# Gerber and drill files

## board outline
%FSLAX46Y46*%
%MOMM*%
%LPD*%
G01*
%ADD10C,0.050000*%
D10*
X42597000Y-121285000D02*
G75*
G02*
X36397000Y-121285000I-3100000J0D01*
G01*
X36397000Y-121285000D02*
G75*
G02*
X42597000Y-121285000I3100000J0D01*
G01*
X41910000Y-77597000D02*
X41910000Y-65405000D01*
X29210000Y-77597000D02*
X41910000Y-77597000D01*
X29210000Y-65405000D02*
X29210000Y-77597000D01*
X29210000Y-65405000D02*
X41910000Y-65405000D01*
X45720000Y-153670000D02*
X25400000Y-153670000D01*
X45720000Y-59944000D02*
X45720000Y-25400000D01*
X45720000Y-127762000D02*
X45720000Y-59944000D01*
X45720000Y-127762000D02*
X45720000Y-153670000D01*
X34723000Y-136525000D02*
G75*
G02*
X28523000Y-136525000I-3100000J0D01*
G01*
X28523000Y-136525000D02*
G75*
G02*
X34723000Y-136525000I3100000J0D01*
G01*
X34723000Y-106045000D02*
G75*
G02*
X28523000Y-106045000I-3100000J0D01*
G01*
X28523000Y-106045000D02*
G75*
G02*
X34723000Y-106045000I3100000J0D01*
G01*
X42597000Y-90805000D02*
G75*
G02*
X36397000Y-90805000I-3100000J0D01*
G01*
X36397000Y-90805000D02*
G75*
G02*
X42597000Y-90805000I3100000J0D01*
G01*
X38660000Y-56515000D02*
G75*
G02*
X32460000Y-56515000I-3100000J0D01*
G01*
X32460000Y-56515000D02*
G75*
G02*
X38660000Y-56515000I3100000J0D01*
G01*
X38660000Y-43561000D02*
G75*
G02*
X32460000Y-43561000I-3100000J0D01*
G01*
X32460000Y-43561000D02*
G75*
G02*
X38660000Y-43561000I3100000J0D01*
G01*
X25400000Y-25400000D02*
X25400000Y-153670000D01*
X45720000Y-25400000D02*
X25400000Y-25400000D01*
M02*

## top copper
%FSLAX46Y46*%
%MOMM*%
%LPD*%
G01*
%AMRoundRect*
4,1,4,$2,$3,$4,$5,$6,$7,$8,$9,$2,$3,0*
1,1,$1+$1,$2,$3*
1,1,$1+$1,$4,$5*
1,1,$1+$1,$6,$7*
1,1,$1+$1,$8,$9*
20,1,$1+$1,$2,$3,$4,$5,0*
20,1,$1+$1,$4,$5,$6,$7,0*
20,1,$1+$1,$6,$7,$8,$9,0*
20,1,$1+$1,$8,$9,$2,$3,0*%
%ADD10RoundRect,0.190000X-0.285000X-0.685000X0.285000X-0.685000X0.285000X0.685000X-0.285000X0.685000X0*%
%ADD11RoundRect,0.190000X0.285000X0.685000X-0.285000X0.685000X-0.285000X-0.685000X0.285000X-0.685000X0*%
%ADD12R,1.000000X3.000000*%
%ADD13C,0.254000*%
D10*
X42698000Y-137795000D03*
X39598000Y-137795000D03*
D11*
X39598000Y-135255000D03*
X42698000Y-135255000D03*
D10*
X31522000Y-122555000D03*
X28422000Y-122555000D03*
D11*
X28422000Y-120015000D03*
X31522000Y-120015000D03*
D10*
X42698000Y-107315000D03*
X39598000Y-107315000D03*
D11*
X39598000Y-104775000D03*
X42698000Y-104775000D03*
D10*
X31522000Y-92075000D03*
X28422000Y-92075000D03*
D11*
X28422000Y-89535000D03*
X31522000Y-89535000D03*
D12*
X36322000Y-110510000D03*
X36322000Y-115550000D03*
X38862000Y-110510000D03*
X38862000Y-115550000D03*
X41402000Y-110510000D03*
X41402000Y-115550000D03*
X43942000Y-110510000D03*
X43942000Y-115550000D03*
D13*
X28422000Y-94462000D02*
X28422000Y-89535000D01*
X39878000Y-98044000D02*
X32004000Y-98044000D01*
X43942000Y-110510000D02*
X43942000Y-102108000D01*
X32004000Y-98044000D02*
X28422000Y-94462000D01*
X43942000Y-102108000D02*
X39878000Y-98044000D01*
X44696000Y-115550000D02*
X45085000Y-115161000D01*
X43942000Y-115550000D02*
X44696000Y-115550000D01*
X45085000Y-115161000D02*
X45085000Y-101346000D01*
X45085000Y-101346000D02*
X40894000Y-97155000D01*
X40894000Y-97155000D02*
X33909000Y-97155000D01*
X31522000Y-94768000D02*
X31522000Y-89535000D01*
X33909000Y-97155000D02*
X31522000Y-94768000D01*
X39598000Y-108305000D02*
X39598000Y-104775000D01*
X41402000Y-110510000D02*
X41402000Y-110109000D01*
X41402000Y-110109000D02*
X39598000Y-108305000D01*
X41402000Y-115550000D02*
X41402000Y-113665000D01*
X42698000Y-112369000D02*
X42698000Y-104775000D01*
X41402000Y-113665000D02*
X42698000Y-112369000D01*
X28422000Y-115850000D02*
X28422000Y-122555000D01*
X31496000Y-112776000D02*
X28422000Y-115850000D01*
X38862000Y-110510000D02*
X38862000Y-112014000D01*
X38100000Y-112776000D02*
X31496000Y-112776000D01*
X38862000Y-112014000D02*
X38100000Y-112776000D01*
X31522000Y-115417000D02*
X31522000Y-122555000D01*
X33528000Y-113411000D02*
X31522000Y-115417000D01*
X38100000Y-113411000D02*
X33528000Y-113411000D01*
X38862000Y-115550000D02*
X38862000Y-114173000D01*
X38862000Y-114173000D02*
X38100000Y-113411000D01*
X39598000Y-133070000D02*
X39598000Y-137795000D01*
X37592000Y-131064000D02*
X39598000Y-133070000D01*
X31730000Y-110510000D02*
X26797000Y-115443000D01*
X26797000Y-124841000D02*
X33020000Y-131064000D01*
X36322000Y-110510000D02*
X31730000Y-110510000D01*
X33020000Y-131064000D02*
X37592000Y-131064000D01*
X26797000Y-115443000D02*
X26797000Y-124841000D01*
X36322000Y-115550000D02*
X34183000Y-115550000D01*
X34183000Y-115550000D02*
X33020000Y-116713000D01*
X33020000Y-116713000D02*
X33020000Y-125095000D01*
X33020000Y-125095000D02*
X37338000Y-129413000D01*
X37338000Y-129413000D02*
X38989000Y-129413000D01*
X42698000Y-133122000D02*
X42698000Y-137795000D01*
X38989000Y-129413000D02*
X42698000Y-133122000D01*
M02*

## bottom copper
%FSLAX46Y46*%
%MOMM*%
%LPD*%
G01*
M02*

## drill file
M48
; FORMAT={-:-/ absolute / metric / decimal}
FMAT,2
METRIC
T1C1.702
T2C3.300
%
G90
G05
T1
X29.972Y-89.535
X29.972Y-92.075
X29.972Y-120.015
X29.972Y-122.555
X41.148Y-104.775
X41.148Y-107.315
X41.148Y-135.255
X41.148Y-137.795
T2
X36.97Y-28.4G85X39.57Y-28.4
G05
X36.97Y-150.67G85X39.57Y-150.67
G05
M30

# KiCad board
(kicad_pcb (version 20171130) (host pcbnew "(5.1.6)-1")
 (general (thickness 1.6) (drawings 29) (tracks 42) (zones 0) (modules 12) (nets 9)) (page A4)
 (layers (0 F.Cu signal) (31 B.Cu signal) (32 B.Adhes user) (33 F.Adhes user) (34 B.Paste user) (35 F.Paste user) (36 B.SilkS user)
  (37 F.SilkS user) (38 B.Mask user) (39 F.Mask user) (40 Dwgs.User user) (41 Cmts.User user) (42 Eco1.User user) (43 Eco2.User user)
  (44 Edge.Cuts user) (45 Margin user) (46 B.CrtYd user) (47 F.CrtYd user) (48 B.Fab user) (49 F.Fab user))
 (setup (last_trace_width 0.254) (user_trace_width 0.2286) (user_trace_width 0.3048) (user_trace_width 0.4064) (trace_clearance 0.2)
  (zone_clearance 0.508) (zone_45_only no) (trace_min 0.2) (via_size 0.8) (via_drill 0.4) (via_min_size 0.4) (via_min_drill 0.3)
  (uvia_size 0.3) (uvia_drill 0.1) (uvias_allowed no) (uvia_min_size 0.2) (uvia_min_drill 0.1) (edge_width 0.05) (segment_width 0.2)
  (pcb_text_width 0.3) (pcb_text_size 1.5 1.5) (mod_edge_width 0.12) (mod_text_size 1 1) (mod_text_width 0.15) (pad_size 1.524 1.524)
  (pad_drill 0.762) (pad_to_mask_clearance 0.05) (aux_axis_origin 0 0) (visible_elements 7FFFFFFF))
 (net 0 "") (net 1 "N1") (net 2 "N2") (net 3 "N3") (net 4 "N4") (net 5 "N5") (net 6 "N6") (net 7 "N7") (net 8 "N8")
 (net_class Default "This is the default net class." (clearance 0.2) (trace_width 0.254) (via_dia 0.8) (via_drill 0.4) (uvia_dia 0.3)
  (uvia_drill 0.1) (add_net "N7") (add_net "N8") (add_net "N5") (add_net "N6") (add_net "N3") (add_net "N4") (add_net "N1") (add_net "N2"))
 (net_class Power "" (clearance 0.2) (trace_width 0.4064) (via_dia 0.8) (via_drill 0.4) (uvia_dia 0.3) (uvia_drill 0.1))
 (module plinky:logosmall (layer F.Cu) (at 35.687 34.417)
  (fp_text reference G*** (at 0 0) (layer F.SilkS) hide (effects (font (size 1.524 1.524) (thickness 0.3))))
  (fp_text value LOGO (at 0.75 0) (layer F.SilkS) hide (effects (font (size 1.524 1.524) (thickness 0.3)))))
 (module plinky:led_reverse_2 (layer F.Cu) (at 41.148 137.795)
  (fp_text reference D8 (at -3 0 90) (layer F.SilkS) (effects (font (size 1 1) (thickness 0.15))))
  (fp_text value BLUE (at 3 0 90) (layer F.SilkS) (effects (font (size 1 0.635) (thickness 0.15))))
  (pad "" np_thru_hole oval (at 0 0) (size 1.7018 1.7018) (drill oval 1.7018) (layers *.Cu *.Mask))
  (pad 2 smd roundrect (at 1.55 0) (size 0.95 1.75) (layers F.Cu F.Paste F.Mask) (roundrect_rratio 0.2) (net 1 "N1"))
  (pad 1 smd roundrect (at -1.55 0) (size 0.95 1.75) (layers F.Cu F.Paste F.Mask) (roundrect_rratio 0.2) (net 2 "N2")))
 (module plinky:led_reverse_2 (layer F.Cu) (at 41.148 135.255 180)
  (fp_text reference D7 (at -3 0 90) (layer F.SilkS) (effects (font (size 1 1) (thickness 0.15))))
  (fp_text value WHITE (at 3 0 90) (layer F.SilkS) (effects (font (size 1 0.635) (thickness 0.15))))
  (pad "" np_thru_hole oval (at 0 0 180) (size 1.7018 1.7018) (drill oval 1.7018) (layers *.Cu *.Mask))
  (pad 2 smd roundrect (at 1.55 0 180) (size 0.95 1.75) (layers F.Cu F.Paste F.Mask) (roundrect_rratio 0.2) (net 2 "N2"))
  (pad 1 smd roundrect (at -1.55 0 180) (size 0.95 1.75) (layers F.Cu F.Paste F.Mask) (roundrect_rratio 0.2) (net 1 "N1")))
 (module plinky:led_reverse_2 (layer F.Cu) (at 29.972 122.555)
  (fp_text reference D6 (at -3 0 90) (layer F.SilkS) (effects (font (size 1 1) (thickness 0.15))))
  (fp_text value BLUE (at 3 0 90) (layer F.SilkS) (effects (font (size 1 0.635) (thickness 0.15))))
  (pad "" np_thru_hole oval (at 0 0) (size 1.7018 1.7018) (drill oval 1.7018) (layers *.Cu *.Mask))
  (pad 2 smd roundrect (at 1.55 0) (size 0.95 1.75) (layers F.Cu F.Paste F.Mask) (roundrect_rratio 0.2) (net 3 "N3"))
  (pad 1 smd roundrect (at -1.55 0) (size 0.95 1.75) (layers F.Cu F.Paste F.Mask) (roundrect_rratio 0.2) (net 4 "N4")))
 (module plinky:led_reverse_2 (layer F.Cu) (at 29.972 120.015 180)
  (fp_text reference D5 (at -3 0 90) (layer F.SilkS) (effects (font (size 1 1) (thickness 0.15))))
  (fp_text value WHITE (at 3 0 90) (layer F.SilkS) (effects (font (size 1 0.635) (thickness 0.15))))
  (pad "" np_thru_hole oval (at 0 0 180) (size 1.7018 1.7018) (drill oval 1.7018) (layers *.Cu *.Mask))
  (pad 2 smd roundrect (at 1.55 0 180) (size 0.95 1.75) (layers F.Cu F.Paste F.Mask) (roundrect_rratio 0.2) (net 4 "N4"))
  (pad 1 smd roundrect (at -1.55 0 180) (size 0.95 1.75) (layers F.Cu F.Paste F.Mask) (roundrect_rratio 0.2) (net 3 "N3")))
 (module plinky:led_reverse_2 (layer F.Cu) (at 41.148 107.315)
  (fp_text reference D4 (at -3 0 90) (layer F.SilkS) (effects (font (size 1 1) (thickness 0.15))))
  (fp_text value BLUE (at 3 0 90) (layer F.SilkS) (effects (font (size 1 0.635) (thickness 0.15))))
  (pad "" np_thru_hole oval (at 0 0) (size 1.7018 1.7018) (drill oval 1.7018) (layers *.Cu *.Mask))
  (pad 2 smd roundrect (at 1.55 0) (size 0.95 1.75) (layers F.Cu F.Paste F.Mask) (roundrect_rratio 0.2) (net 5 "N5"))
  (pad 1 smd roundrect (at -1.55 0) (size 0.95 1.75) (layers F.Cu F.Paste F.Mask) (roundrect_rratio 0.2) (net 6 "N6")))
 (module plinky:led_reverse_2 (layer F.Cu) (at 41.148 104.775 180)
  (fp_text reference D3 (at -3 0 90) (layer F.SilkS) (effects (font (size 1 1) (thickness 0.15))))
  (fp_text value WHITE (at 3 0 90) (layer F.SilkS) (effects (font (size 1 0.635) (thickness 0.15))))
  (pad "" np_thru_hole oval (at 0 0 180) (size 1.7018 1.7018) (drill oval 1.7018) (layers *.Cu *.Mask))
  (pad 2 smd roundrect (at 1.55 0 180) (size 0.95 1.75) (layers F.Cu F.Paste F.Mask) (roundrect_rratio 0.2) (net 6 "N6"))
  (pad 1 smd roundrect (at -1.55 0 180) (size 0.95 1.75) (layers F.Cu F.Paste F.Mask) (roundrect_rratio 0.2) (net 5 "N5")))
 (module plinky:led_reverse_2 (layer F.Cu) (at 29.972 92.075)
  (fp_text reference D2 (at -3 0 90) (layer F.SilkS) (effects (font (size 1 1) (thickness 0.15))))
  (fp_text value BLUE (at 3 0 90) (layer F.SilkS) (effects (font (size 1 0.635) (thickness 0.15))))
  (pad "" np_thru_hole oval (at 0 0) (size 1.7018 1.7018) (drill oval 1.7018) (layers *.Cu *.Mask))
  (pad 2 smd roundrect (at 1.55 0) (size 0.95 1.75) (layers F.Cu F.Paste F.Mask) (roundrect_rratio 0.2) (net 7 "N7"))
  (pad 1 smd roundrect (at -1.55 0) (size 0.95 1.75) (layers F.Cu F.Paste F.Mask) (roundrect_rratio 0.2) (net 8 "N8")))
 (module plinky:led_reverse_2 (layer F.Cu) (at 29.972 89.535 180)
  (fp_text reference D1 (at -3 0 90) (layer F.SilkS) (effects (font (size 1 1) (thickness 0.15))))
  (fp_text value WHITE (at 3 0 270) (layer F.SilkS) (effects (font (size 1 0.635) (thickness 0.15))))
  (pad "" np_thru_hole oval (at 0 0 180) (size 1.7018 1.7018) (drill oval 1.7018) (layers *.Cu *.Mask))
  (pad 2 smd roundrect (at 1.55 0 180) (size 0.95 1.75) (layers F.Cu F.Paste F.Mask) (roundrect_rratio 0.2) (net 8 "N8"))
  (pad 1 smd roundrect (at -1.55 0 180) (size 0.95 1.75) (layers F.Cu F.Paste F.Mask) (roundrect_rratio 0.2) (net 7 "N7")))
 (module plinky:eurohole (layer F.Cu) (at 38.27 28.4)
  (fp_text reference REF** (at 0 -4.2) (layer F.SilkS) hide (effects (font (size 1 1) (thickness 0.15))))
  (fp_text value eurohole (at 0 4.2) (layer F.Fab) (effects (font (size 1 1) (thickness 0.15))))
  (pad "" np_thru_hole oval (at 0 0) (size 5.9 3.3) (drill oval 5.9 3.3) (layers *.Cu *.Mask)))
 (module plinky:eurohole (layer F.Cu) (at 38.27 150.67)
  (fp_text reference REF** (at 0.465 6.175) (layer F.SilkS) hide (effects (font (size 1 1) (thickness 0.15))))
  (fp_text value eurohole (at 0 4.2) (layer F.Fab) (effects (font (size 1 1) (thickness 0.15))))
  (pad "" np_thru_hole oval (at 0 0) (size 5.9 3.3) (drill oval 5.9 3.3) (layers *.Cu *.Mask)))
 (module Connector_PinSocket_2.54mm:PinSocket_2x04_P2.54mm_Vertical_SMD (layer F.Cu) (at 40.132 113.03 270)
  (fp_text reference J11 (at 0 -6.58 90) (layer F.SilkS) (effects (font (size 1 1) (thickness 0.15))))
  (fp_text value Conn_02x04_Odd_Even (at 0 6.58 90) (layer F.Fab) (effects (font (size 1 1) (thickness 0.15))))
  (pad 8 smd rect (at -2.52 3.81 270) (size 3 1) (layers F.Cu F.Paste F.Mask) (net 2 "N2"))
  (pad 7 smd rect (at 2.52 3.81 270) (size 3 1) (layers F.Cu F.Paste F.Mask) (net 1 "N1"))
  (pad 6 smd rect (at -2.52 1.27 270) (size 3 1) (layers F.Cu F.Paste F.Mask) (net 4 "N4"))
  (pad 5 smd rect (at 2.52 1.27 270) (size 3 1) (layers F.Cu F.Paste F.Mask) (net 3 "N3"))
  (pad 4 smd rect (at -2.52 -1.27 270) (size 3 1) (layers F.Cu F.Paste F.Mask) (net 6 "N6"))
  (pad 3 smd rect (at 2.52 -1.27 270) (size 3 1) (layers F.Cu F.Paste F.Mask) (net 5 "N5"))
  (pad 2 smd rect (at -2.52 -3.81 270) (size 3 1) (layers F.Cu F.Paste F.Mask) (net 8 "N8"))
  (pad 1 smd rect (at 2.52 -3.81 270) (size 3 1) (layers F.Cu F.Paste F.Mask) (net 7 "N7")))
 (gr_circle (center 39.497 121.285) (end 36.397 121.285) (layer Edge.Cuts) (width 0.05))
 (gr_line (start 41.91 77.597) (end 41.91 65.405) (layer Edge.Cuts) (width 0.05))
 (gr_line (start 29.21 77.597) (end 41.91 77.597) (layer Edge.Cuts) (width 0.05))
 (gr_line (start 29.21 65.405) (end 29.21 77.597) (layer Edge.Cuts) (width 0.05))
 (gr_line (start 29.21 65.405) (end 41.91 65.405) (layer Edge.Cuts) (width 0.05))
 (gr_line (start 45.72 153.67) (end 25.4 153.67) (layer Edge.Cuts) (width 0.05))
 (gr_line (start 45.72 59.944) (end 45.72 25.4) (layer Edge.Cuts) (width 0.05))
 (gr_line (start 45.72 127.762) (end 45.72 59.944) (layer Edge.Cuts) (width 0.05))
 (gr_line (start 45.72 127.762) (end 45.72 153.67) (layer Edge.Cuts) (width 0.05))
 (gr_circle (center 31.623 136.525) (end 28.523 136.525) (layer Edge.Cuts) (width 0.05))
 (gr_circle (center 31.623 106.045) (end 28.523 106.045) (layer Edge.Cuts) (width 0.05))
 (gr_circle (center 39.497 90.805) (end 36.397 90.805) (layer Edge.Cuts) (width 0.05))
 (gr_circle (center 35.56 56.515) (end 32.46 56.515) (layer Edge.Cuts) (width 0.05))
 (gr_circle (center 35.56 43.561) (end 32.46 43.561) (layer Edge.Cuts) (width 0.05))
 (gr_line (start 25.4 25.4) (end 25.4 153.67) (layer Edge.Cuts) (width 0.05))
 (gr_line (start 45.72 25.4) (end 25.4 25.4) (layer Edge.Cuts) (width 0.05))
 (segment (start 28.422 94.462) (end 28.422 89.535) (width 0.254) (layer F.Cu) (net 8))
 (segment (start 39.878 98.044) (end 32.004 98.044) (width 0.254) (layer F.Cu) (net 8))
 (segment (start 43.942 110.51) (end 43.942 102.108) (width 0.254) (layer F.Cu) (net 8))
 (segment (start 32.004 98.044) (end 28.422 94.462) (width 0.254) (layer F.Cu) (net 8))
 (segment (start 43.942 102.108) (end 39.878 98.044) (width 0.254) (layer F.Cu) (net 8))
 (segment (start 44.696 115.55) (end 45.085 115.161) (width 0.254) (layer F.Cu) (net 7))
 (segment (start 43.942 115.55) (end 44.696 115.55) (width 0.254) (layer F.Cu) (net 7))
 (segment (start 45.085 115.161) (end 45.085 101.346) (width 0.254) (layer F.Cu) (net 7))
 (segment (start 45.085 101.346) (end 40.894 97.155) (width 0.254) (layer F.Cu) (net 7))
 (segment (start 40.894 97.155) (end 33.909 97.155) (width 0.254) (layer F.Cu) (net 7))
 (segment (start 31.522 94.768) (end 31.522 89.535) (width 0.254) (layer F.Cu) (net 7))
 (segment (start 33.909 97.155) (end 31.522 94.768) (width 0.254) (layer F.Cu) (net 7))
 (segment (start 39.598 108.305) (end 39.598 104.775) (width 0.254) (layer F.Cu) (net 6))
 (segment (start 41.402 110.51) (end 41.402 110.109) (width 0.254) (layer F.Cu) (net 6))
 (segment (start 41.402 110.109) (end 39.598 108.305) (width 0.254) (layer F.Cu) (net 6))
 (segment (start 41.402 115.55) (end 41.402 113.665) (width 0.254) (layer F.Cu) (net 5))
 (segment (start 42.698 112.369) (end 42.698 104.775) (width 0.254) (layer F.Cu) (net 5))
 (segment (start 41.402 113.665) (end 42.698 112.369) (width 0.254) (layer F.Cu) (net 5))
 (segment (start 28.422 115.85) (end 28.422 122.555) (width 0.254) (layer F.Cu) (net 4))
 (segment (start 31.496 112.776) (end 28.422 115.85) (width 0.254) (layer F.Cu) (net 4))
 (segment (start 38.862 110.51) (end 38.862 112.014) (width 0.254) (layer F.Cu) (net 4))
 (segment (start 38.1 112.776) (end 31.496 112.776) (width 0.254) (layer F.Cu) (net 4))
 (segment (start 38.862 112.014) (end 38.1 112.776) (width 0.254) (layer F.Cu) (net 4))
 (segment (start 31.522 115.417) (end 31.522 122.555) (width 0.254) (layer F.Cu) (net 3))
 (segment (start 33.528 113.411) (end 31.522 115.417) (width 0.254) (layer F.Cu) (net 3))
 (segment (start 38.1 113.411) (end 33.528 113.411) (width 0.254) (layer F.Cu) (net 3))
 (segment (start 38.862 115.55) (end 38.862 114.173) (width 0.254) (layer F.Cu) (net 3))
 (segment (start 38.862 114.173) (end 38.1 113.411) (width 0.254) (layer F.Cu) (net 3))
 (segment (start 39.598 133.07) (end 39.598 137.795) (width 0.254) (layer F.Cu) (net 2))
 (segment (start 37.592 131.064) (end 39.598 133.07) (width 0.254) (layer F.Cu) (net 2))
 (segment (start 31.73 110.51) (end 26.797 115.443) (width 0.254) (layer F.Cu) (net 2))
 (segment (start 26.797 124.841) (end 33.02 131.064) (width 0.254) (layer F.Cu) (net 2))
 (segment (start 36.322 110.51) (end 31.73 110.51) (width 0.254) (layer F.Cu) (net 2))
 (segment (start 33.02 131.064) (end 37.592 131.064) (width 0.254) (layer F.Cu) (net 2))
 (segment (start 26.797 115.443) (end 26.797 124.841) (width 0.254) (layer F.Cu) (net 2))
 (segment (start 36.322 115.55) (end 34.183 115.55) (width 0.254) (layer F.Cu) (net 1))
 (segment (start 34.183 115.55) (end 33.02 116.713) (width 0.254) (layer F.Cu) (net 1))
 (segment (start 33.02 116.713) (end 33.02 125.095) (width 0.254) (layer F.Cu) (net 1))
 (segment (start 33.02 125.095) (end 37.338 129.413) (width 0.254) (layer F.Cu) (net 1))
 (segment (start 37.338 129.413) (end 38.989 129.413) (width 0.254) (layer F.Cu) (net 1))
 (segment (start 42.698 133.122) (end 42.698 137.795) (width 0.254) (layer F.Cu) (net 1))
 (segment (start 38.989 129.413) (end 42.698 133.122) (width 0.254) (layer F.Cu) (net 1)))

